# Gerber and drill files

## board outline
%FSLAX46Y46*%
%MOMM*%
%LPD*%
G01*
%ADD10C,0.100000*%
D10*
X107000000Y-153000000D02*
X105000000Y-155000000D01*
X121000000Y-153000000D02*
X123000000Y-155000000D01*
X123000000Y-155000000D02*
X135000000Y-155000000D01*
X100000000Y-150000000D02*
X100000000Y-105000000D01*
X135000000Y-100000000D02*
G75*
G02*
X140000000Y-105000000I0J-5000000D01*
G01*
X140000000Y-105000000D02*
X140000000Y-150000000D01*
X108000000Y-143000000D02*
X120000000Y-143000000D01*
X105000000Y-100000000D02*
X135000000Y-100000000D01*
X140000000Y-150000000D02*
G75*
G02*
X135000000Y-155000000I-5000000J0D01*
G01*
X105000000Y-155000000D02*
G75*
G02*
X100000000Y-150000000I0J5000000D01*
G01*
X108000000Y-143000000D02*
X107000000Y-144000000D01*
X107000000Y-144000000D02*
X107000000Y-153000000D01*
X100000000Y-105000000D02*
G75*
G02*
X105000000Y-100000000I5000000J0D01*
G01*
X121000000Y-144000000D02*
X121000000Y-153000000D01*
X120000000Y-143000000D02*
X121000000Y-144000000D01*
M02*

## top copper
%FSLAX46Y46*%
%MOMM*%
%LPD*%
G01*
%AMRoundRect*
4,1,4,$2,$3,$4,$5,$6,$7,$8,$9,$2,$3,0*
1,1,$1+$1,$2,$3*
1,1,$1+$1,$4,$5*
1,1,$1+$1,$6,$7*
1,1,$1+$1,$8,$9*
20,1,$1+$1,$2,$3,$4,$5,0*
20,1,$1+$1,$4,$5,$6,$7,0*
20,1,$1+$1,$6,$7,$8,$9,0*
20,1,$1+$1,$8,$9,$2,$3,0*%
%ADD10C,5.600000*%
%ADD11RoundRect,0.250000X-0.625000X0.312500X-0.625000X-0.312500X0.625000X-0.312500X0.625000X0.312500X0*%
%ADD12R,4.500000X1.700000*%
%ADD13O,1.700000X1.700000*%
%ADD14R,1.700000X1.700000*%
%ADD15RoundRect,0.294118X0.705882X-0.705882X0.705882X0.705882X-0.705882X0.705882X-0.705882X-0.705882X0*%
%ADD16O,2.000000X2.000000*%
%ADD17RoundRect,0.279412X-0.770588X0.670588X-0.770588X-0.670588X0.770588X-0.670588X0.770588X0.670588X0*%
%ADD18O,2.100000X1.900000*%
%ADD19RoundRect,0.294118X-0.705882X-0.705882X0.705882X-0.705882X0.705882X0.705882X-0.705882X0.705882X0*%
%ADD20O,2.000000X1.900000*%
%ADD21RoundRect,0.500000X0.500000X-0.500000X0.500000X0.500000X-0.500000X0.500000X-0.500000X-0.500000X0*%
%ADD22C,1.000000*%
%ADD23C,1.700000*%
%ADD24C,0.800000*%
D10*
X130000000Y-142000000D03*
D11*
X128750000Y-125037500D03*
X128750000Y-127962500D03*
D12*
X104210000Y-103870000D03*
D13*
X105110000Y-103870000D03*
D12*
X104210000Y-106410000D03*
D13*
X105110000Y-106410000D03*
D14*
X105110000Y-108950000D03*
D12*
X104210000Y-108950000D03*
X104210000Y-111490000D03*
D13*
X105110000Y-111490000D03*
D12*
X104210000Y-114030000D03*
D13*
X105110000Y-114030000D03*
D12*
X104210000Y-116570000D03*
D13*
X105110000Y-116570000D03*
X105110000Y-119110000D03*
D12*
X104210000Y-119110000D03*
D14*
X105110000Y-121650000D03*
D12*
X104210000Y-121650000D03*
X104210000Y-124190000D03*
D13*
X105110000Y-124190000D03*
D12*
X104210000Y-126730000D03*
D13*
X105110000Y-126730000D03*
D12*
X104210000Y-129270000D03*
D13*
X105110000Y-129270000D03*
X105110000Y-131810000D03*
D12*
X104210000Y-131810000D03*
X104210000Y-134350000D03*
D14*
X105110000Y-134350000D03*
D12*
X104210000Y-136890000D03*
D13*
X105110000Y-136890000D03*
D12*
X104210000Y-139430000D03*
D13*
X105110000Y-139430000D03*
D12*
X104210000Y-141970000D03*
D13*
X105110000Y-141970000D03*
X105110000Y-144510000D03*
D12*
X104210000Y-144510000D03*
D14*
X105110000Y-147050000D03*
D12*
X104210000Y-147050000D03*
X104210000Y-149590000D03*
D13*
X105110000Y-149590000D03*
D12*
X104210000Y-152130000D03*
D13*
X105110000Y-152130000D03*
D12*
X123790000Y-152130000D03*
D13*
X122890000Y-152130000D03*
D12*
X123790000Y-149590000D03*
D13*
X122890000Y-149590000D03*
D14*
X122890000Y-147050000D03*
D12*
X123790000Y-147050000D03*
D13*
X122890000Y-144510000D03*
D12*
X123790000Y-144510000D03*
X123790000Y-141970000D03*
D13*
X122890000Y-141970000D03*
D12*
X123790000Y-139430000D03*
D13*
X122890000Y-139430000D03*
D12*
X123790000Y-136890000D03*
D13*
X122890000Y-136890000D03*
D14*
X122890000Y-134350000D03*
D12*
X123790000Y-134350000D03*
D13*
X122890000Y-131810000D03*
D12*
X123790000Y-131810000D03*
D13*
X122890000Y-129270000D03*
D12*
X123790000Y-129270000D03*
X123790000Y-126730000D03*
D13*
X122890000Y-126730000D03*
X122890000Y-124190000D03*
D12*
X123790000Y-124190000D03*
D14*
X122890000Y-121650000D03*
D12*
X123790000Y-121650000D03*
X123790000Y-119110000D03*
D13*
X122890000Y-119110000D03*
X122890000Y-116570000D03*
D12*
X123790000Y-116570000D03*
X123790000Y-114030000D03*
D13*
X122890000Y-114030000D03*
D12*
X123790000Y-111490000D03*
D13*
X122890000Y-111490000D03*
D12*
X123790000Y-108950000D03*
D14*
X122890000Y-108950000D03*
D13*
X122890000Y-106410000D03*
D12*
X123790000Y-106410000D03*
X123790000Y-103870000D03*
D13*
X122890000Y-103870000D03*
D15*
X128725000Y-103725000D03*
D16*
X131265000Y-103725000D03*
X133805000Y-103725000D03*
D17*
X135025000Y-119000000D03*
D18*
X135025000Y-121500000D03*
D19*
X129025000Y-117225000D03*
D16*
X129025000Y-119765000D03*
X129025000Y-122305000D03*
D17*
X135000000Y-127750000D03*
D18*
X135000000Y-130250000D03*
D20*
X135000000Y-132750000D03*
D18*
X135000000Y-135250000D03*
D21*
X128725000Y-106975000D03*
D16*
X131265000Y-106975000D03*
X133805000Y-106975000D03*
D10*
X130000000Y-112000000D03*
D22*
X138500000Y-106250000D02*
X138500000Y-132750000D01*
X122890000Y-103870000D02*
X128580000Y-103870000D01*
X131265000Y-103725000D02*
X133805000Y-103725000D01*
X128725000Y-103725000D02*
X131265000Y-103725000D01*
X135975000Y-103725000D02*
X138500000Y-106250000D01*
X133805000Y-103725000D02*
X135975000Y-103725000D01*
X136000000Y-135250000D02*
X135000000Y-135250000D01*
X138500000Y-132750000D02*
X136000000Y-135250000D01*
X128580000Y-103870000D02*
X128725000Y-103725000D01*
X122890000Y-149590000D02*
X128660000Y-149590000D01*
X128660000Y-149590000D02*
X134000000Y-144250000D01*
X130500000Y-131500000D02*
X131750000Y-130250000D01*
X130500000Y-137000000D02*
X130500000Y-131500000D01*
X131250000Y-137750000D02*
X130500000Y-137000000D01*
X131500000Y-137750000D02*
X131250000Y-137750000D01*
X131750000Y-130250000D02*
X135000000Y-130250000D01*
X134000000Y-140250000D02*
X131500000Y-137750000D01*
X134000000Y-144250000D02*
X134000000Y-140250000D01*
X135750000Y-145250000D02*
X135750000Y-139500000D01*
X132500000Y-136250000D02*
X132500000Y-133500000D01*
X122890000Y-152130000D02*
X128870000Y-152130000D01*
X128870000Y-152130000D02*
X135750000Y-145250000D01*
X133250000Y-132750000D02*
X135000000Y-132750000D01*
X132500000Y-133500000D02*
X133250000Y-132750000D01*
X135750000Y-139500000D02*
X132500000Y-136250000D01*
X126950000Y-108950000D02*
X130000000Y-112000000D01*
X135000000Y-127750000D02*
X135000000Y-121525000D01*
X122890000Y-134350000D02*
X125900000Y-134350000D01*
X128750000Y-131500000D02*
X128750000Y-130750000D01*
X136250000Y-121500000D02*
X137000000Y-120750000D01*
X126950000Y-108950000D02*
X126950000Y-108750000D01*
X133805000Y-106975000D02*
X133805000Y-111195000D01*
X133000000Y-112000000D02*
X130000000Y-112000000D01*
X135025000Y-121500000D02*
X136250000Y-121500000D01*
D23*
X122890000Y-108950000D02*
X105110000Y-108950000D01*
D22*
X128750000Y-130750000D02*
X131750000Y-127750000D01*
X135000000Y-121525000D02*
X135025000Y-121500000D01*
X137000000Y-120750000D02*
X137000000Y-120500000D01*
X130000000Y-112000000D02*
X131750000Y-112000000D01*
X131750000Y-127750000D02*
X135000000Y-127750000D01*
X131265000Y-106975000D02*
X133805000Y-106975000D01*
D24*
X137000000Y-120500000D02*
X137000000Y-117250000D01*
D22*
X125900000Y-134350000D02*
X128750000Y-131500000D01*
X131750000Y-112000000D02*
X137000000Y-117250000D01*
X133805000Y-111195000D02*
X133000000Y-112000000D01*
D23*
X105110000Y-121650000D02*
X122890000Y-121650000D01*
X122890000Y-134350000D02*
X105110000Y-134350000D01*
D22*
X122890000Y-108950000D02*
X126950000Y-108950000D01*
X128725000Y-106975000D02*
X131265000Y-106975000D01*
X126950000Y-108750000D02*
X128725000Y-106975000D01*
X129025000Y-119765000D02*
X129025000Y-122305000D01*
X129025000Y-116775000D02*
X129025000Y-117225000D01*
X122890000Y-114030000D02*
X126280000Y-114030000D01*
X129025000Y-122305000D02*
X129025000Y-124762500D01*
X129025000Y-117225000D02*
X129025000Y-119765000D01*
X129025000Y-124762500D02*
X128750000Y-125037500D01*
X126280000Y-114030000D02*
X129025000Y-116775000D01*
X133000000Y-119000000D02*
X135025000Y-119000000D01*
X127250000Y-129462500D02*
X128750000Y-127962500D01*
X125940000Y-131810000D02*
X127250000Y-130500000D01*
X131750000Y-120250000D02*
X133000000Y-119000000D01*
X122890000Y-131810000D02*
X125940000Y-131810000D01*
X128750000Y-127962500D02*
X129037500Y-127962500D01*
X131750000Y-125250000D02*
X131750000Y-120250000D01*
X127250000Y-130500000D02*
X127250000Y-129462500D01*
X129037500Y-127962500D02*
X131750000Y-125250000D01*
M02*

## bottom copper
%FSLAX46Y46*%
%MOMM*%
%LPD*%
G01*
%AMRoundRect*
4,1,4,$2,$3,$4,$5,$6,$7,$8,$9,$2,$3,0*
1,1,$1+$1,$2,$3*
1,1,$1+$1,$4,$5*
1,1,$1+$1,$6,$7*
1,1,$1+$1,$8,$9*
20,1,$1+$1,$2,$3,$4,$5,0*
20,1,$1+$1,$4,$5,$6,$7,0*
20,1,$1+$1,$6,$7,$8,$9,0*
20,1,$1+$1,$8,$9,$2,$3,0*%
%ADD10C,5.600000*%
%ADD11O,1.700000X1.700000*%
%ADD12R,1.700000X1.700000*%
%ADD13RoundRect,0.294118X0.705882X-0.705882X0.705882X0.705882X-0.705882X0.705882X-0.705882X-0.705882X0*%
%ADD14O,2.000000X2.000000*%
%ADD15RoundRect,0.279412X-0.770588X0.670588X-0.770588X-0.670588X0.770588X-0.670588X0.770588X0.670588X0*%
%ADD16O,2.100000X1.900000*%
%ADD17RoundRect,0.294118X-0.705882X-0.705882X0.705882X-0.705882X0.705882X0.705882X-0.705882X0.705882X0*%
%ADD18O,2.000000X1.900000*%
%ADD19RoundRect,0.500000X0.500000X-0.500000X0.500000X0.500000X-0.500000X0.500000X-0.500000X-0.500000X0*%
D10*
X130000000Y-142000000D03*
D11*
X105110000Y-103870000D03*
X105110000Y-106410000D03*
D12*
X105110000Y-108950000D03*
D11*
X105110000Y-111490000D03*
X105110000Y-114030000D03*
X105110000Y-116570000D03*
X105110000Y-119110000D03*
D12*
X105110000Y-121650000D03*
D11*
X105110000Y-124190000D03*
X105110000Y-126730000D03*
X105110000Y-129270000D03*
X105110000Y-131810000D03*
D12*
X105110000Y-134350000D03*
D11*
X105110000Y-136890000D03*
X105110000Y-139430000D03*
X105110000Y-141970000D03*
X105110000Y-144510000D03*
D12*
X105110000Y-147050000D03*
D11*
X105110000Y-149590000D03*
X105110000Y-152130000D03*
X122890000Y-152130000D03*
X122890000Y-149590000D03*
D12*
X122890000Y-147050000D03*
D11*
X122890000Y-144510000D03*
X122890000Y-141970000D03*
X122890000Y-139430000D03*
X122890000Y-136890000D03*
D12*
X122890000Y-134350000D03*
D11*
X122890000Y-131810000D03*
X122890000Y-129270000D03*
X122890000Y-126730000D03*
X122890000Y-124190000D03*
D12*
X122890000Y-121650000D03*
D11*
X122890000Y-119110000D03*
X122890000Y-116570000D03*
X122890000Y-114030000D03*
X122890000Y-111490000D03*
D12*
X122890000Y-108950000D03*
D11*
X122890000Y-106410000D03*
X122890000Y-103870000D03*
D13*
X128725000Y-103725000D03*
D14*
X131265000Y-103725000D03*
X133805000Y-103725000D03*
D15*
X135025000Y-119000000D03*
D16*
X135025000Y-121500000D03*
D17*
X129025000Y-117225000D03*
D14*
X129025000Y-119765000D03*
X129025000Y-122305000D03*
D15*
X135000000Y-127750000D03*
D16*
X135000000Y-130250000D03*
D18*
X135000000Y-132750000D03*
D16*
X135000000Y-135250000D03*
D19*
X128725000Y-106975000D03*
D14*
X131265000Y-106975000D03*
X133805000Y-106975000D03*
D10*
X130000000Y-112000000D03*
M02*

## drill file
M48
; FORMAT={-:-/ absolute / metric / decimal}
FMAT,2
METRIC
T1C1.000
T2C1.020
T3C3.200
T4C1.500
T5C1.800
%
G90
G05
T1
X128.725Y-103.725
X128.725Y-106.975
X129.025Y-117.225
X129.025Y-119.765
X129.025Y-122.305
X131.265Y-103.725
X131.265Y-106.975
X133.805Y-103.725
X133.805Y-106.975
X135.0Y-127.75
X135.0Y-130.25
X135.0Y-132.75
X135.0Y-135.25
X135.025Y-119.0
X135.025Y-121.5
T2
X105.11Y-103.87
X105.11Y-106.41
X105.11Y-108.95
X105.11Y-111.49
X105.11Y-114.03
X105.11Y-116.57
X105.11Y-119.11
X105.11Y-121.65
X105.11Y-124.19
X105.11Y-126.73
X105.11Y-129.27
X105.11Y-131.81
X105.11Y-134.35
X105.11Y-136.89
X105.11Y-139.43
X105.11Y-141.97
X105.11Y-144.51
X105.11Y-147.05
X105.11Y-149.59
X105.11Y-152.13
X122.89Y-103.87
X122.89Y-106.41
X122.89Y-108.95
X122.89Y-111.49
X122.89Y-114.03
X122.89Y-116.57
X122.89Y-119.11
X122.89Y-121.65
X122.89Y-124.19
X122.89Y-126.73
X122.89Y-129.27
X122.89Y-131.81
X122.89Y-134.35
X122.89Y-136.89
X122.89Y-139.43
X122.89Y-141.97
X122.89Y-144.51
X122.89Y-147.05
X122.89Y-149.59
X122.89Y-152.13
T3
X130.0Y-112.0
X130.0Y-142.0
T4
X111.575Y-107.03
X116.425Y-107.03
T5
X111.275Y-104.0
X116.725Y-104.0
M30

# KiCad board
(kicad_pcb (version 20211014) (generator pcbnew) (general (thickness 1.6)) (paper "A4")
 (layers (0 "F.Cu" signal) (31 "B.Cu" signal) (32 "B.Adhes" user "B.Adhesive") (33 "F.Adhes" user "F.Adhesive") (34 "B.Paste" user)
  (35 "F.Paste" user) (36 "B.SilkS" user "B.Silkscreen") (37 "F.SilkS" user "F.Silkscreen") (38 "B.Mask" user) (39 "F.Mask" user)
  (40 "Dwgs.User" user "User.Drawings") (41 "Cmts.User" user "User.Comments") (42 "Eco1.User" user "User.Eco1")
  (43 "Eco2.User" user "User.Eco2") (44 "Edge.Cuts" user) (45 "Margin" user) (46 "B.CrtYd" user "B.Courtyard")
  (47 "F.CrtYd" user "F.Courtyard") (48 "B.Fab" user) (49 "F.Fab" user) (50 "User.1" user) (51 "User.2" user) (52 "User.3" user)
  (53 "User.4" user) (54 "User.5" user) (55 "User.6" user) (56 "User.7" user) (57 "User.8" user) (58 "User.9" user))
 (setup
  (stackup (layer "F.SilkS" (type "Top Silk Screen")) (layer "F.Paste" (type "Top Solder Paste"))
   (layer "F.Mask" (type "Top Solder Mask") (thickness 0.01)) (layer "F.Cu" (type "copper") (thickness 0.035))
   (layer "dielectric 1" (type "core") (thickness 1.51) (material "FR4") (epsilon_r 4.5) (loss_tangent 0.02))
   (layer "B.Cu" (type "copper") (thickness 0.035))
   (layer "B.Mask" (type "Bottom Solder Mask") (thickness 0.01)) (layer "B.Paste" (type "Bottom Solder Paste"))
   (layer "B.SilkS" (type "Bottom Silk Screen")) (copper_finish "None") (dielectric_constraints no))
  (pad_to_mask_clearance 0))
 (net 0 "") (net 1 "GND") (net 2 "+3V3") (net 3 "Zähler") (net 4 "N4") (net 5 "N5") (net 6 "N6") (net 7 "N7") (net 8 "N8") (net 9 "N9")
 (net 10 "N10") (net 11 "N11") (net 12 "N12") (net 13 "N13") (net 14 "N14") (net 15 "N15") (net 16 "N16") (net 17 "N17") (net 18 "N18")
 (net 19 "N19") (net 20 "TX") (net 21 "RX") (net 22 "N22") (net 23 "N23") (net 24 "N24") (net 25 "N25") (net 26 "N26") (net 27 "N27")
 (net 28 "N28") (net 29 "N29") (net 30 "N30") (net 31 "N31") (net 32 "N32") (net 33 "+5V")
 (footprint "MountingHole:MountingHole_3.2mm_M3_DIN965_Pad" (layer "F.Cu") (at 130 142)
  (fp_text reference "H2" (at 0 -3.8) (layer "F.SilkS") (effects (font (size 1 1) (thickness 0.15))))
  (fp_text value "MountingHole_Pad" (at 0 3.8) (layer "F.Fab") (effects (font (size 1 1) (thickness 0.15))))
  (pad "1" thru_hole circle (at 0 0) (size 5.6 5.6) (drill 3.2) (layers *.Cu *.Mask) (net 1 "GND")))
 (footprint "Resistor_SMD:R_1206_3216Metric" (layer "F.Cu") (at 128.75 126.5 -90)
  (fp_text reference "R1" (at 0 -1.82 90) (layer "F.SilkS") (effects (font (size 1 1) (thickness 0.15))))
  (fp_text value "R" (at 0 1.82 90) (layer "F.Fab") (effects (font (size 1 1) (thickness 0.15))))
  (pad "1" smd roundrect (at -1.4625 0 270) (size 1.125 1.75) (layers "F.Cu" "F.Paste" "F.Mask") (roundrect_rratio 0.222222) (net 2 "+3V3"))
  (pad "2" smd roundrect (at 1.4625 0 270) (size 1.125 1.75) (layers "F.Cu" "F.Paste" "F.Mask") (roundrect_rratio 0.222222) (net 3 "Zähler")))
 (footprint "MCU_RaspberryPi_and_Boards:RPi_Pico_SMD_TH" (layer "F.Cu") (at 114 128)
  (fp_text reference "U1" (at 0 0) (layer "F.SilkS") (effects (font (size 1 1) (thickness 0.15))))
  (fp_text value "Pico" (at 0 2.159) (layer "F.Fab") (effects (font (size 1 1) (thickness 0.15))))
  (pad "" np_thru_hole oval (at -2.425 -20.97) (size 1.5 1.5) (drill 1.5) (layers *.Cu *.Mask))
  (pad "" np_thru_hole oval (at 2.425 -20.97) (size 1.5 1.5) (drill 1.5) (layers *.Cu *.Mask))
  (pad "" np_thru_hole oval (at -2.725 -24) (size 1.8 1.8) (drill 1.8) (layers *.Cu *.Mask))
  (pad "" np_thru_hole oval (at 2.725 -24) (size 1.8 1.8) (drill 1.8) (layers *.Cu *.Mask))
  (pad "1" smd rect (at -8.89 -24.13) (size 4.5 1.7) (drill (offset -0.9 0)) (layers "F.Cu" "F.Mask") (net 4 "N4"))
  (pad "1" thru_hole oval (at -8.89 -24.13) (size 1.7 1.7) (drill 1.02) (layers *.Cu *.Mask) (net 4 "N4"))
  (pad "2" smd rect (at -8.89 -21.59) (size 4.5 1.7) (drill (offset -0.9 0)) (layers "F.Cu" "F.Mask") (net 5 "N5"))
  (pad "2" thru_hole oval (at -8.89 -21.59) (size 1.7 1.7) (drill 1.02) (layers *.Cu *.Mask) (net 5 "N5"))
  (pad "3" thru_hole rect (at -8.89 -19.05) (size 1.7 1.7) (drill 1.02) (layers *.Cu *.Mask) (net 1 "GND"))
  (pad "3" smd rect (at -8.89 -19.05) (size 4.5 1.7) (drill (offset -0.9 0)) (layers "F.Cu" "F.Mask") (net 1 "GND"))
  (pad "4" smd rect (at -8.89 -16.51) (size 4.5 1.7) (drill (offset -0.9 0)) (layers "F.Cu" "F.Mask") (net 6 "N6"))
  (pad "4" thru_hole oval (at -8.89 -16.51) (size 1.7 1.7) (drill 1.02) (layers *.Cu *.Mask) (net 6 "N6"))
  (pad "5" smd rect (at -8.89 -13.97) (size 4.5 1.7) (drill (offset -0.9 0)) (layers "F.Cu" "F.Mask") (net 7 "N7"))
  (pad "5" thru_hole oval (at -8.89 -13.97) (size 1.7 1.7) (drill 1.02) (layers *.Cu *.Mask) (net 7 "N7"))
  (pad "6" smd rect (at -8.89 -11.43) (size 4.5 1.7) (drill (offset -0.9 0)) (layers "F.Cu" "F.Mask") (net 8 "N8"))
  (pad "6" thru_hole oval (at -8.89 -11.43) (size 1.7 1.7) (drill 1.02) (layers *.Cu *.Mask) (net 8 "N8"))
  (pad "7" thru_hole oval (at -8.89 -8.89) (size 1.7 1.7) (drill 1.02) (layers *.Cu *.Mask) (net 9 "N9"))
  (pad "7" smd rect (at -8.89 -8.89) (size 4.5 1.7) (drill (offset -0.9 0)) (layers "F.Cu" "F.Mask") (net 9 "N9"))
  (pad "8" thru_hole rect (at -8.89 -6.35) (size 1.7 1.7) (drill 1.02) (layers *.Cu *.Mask) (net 1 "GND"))
  (pad "8" smd rect (at -8.89 -6.35) (size 4.5 1.7) (drill (offset -0.9 0)) (layers "F.Cu" "F.Mask") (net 1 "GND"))
  (pad "9" smd rect (at -8.89 -3.81) (size 4.5 1.7) (drill (offset -0.9 0)) (layers "F.Cu" "F.Mask") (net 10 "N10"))
  (pad "9" thru_hole oval (at -8.89 -3.81) (size 1.7 1.7) (drill 1.02) (layers *.Cu *.Mask) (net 10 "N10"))
  (pad "10" smd rect (at -8.89 -1.27) (size 4.5 1.7) (drill (offset -0.9 0)) (layers "F.Cu" "F.Mask") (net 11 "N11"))
  (pad "10" thru_hole oval (at -8.89 -1.27) (size 1.7 1.7) (drill 1.02) (layers *.Cu *.Mask) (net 11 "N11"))
  (pad "11" smd rect (at -8.89 1.27) (size 4.5 1.7) (drill (offset -0.9 0)) (layers "F.Cu" "F.Mask") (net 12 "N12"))
  (pad "11" thru_hole oval (at -8.89 1.27) (size 1.7 1.7) (drill 1.02) (layers *.Cu *.Mask) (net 12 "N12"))
  (pad "12" thru_hole oval (at -8.89 3.81) (size 1.7 1.7) (drill 1.02) (layers *.Cu *.Mask) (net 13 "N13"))
  (pad "12" smd rect (at -8.89 3.81) (size 4.5 1.7) (drill (offset -0.9 0)) (layers "F.Cu" "F.Mask") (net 13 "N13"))
  (pad "13" smd rect (at -8.89 6.35) (size 4.5 1.7) (drill (offset -0.9 0)) (layers "F.Cu" "F.Mask") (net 1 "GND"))
  (pad "13" thru_hole rect (at -8.89 6.35) (size 1.7 1.7) (drill 1.02) (layers *.Cu *.Mask) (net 1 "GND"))
  (pad "14" smd rect (at -8.89 8.89) (size 4.5 1.7) (drill (offset -0.9 0)) (layers "F.Cu" "F.Mask") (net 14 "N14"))
  (pad "14" thru_hole oval (at -8.89 8.89) (size 1.7 1.7) (drill 1.02) (layers *.Cu *.Mask) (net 14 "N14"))
  (pad "15" smd rect (at -8.89 11.43) (size 4.5 1.7) (drill (offset -0.9 0)) (layers "F.Cu" "F.Mask") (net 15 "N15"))
  (pad "15" thru_hole oval (at -8.89 11.43) (size 1.7 1.7) (drill 1.02) (layers *.Cu *.Mask) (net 15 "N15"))
  (pad "16" smd rect (at -8.89 13.97) (size 4.5 1.7) (drill (offset -0.9 0)) (layers "F.Cu" "F.Mask") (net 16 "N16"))
  (pad "16" thru_hole oval (at -8.89 13.97) (size 1.7 1.7) (drill 1.02) (layers *.Cu *.Mask) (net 16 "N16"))
  (pad "17" thru_hole oval (at -8.89 16.51) (size 1.7 1.7) (drill 1.02) (layers *.Cu *.Mask) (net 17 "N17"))
  (pad "17" smd rect (at -8.89 16.51) (size 4.5 1.7) (drill (offset -0.9 0)) (layers "F.Cu" "F.Mask") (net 17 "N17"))
  (pad "18" thru_hole rect (at -8.89 19.05) (size 1.7 1.7) (drill 1.02) (layers *.Cu *.Mask) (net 1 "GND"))
  (pad "18" smd rect (at -8.89 19.05) (size 4.5 1.7) (drill (offset -0.9 0)) (layers "F.Cu" "F.Mask") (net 1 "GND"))
  (pad "19" smd rect (at -8.89 21.59) (size 4.5 1.7) (drill (offset -0.9 0)) (layers "F.Cu" "F.Mask") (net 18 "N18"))
  (pad "19" thru_hole oval (at -8.89 21.59) (size 1.7 1.7) (drill 1.02) (layers *.Cu *.Mask) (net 18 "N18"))
  (pad "20" smd rect (at -8.89 24.13) (size 4.5 1.7) (drill (offset -0.9 0)) (layers "F.Cu" "F.Mask") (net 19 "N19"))
  (pad "20" thru_hole oval (at -8.89 24.13) (size 1.7 1.7) (drill 1.02) (layers *.Cu *.Mask) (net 19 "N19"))
  (pad "21" smd rect (at 8.89 24.13) (size 4.5 1.7) (drill (offset 0.9 0)) (layers "F.Cu" "F.Mask") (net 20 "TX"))
  (pad "21" thru_hole oval (at 8.89 24.13) (size 1.7 1.7) (drill 1.02) (layers *.Cu *.Mask) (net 20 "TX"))
  (pad "22" smd rect (at 8.89 21.59) (size 4.5 1.7) (drill (offset 0.9 0)) (layers "F.Cu" "F.Mask") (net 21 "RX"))
  (pad "22" thru_hole oval (at 8.89 21.59) (size 1.7 1.7) (drill 1.02) (layers *.Cu *.Mask) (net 21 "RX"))
  (pad "23" thru_hole rect (at 8.89 19.05) (size 1.7 1.7) (drill 1.02) (layers *.Cu *.Mask) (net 1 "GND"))
  (pad "23" smd rect (at 8.89 19.05) (size 4.5 1.7) (drill (offset 0.9 0)) (layers "F.Cu" "F.Mask") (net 1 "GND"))
  (pad "24" thru_hole oval (at 8.89 16.51) (size 1.7 1.7) (drill 1.02) (layers *.Cu *.Mask) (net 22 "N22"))
  (pad "24" smd rect (at 8.89 16.51) (size 4.5 1.7) (drill (offset 0.9 0)) (layers "F.Cu" "F.Mask") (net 22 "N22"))
  (pad "25" smd rect (at 8.89 13.97) (size 4.5 1.7) (drill (offset 0.9 0)) (layers "F.Cu" "F.Mask") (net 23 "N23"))
  (pad "25" thru_hole oval (at 8.89 13.97) (size 1.7 1.7) (drill 1.02) (layers *.Cu *.Mask) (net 23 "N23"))
  (pad "26" smd rect (at 8.89 11.43) (size 4.5 1.7) (drill (offset 0.9 0)) (layers "F.Cu" "F.Mask") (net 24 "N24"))
  (pad "26" thru_hole oval (at 8.89 11.43) (size 1.7 1.7) (drill 1.02) (layers *.Cu *.Mask) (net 24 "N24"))
  (pad "27" smd rect (at 8.89 8.89) (size 4.5 1.7) (drill (offset 0.9 0)) (layers "F.Cu" "F.Mask") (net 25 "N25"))
  (pad "27" thru_hole oval (at 8.89 8.89) (size 1.7 1.7) (drill 1.02) (layers *.Cu *.Mask) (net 25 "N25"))
  (pad "28" thru_hole rect (at 8.89 6.35) (size 1.7 1.7) (drill 1.02) (layers *.Cu *.Mask) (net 1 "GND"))
  (pad "28" smd rect (at 8.89 6.35) (size 4.5 1.7) (drill (offset 0.9 0)) (layers "F.Cu" "F.Mask") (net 1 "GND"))
  (pad "29" thru_hole oval (at 8.89 3.81) (size 1.7 1.7) (drill 1.02) (layers *.Cu *.Mask) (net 3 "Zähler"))
  (pad "29" smd rect (at 8.89 3.81) (size 4.5 1.7) (drill (offset 0.9 0)) (layers "F.Cu" "F.Mask") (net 3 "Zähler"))
  (pad "30" thru_hole oval (at 8.89 1.27) (size 1.7 1.7) (drill 1.02) (layers *.Cu *.Mask) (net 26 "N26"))
  (pad "30" smd rect (at 8.89 1.27) (size 4.5 1.7) (drill (offset 0.9 0)) (layers "F.Cu" "F.Mask") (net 26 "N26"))
  (pad "31" smd rect (at 8.89 -1.27) (size 4.5 1.7) (drill (offset 0.9 0)) (layers "F.Cu" "F.Mask") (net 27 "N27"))
  (pad "31" thru_hole oval (at 8.89 -1.27) (size 1.7 1.7) (drill 1.02) (layers *.Cu *.Mask) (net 27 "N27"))
  (pad "32" thru_hole oval (at 8.89 -3.81) (size 1.7 1.7) (drill 1.02) (layers *.Cu *.Mask) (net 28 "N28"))
  (pad "32" smd rect (at 8.89 -3.81) (size 4.5 1.7) (drill (offset 0.9 0)) (layers "F.Cu" "F.Mask") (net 28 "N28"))
  (pad "33" thru_hole rect (at 8.89 -6.35) (size 1.7 1.7) (drill 1.02) (layers *.Cu *.Mask) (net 1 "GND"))
  (pad "33" smd rect (at 8.89 -6.35) (size 4.5 1.7) (drill (offset 0.9 0)) (layers "F.Cu" "F.Mask") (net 1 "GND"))
  (pad "34" smd rect (at 8.89 -8.89) (size 4.5 1.7) (drill (offset 0.9 0)) (layers "F.Cu" "F.Mask") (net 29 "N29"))
  (pad "34" thru_hole oval (at 8.89 -8.89) (size 1.7 1.7) (drill 1.02) (layers *.Cu *.Mask) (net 29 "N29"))
  (pad "35" thru_hole oval (at 8.89 -11.43) (size 1.7 1.7) (drill 1.02) (layers *.Cu *.Mask) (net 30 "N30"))
  (pad "35" smd rect (at 8.89 -11.43) (size 4.5 1.7) (drill (offset 0.9 0)) (layers "F.Cu" "F.Mask") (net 30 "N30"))
  (pad "36" smd rect (at 8.89 -13.97) (size 4.5 1.7) (drill (offset 0.9 0)) (layers "F.Cu" "F.Mask") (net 2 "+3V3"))
  (pad "36" thru_hole oval (at 8.89 -13.97) (size 1.7 1.7) (drill 1.02) (layers *.Cu *.Mask) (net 2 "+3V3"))
  (pad "37" smd rect (at 8.89 -16.51) (size 4.5 1.7) (drill (offset 0.9 0)) (layers "F.Cu" "F.Mask") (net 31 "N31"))
  (pad "37" thru_hole oval (at 8.89 -16.51) (size 1.7 1.7) (drill 1.02) (layers *.Cu *.Mask) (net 31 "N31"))
  (pad "38" smd rect (at 8.89 -19.05) (size 4.5 1.7) (drill (offset 0.9 0)) (layers "F.Cu" "F.Mask") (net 1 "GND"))
  (pad "38" thru_hole rect (at 8.89 -19.05) (size 1.7 1.7) (drill 1.02) (layers *.Cu *.Mask) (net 1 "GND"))
  (pad "39" thru_hole oval (at 8.89 -21.59) (size 1.7 1.7) (drill 1.02) (layers *.Cu *.Mask) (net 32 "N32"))
  (pad "39" smd rect (at 8.89 -21.59) (size 4.5 1.7) (drill (offset 0.9 0)) (layers "F.Cu" "F.Mask") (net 32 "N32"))
  (pad "40" smd rect (at 8.89 -24.13) (size 4.5 1.7) (drill (offset 0.9 0)) (layers "F.Cu" "F.Mask") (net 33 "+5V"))
  (pad "40" thru_hole oval (at 8.89 -24.13) (size 1.7 1.7) (drill 1.02) (layers *.Cu *.Mask) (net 33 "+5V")))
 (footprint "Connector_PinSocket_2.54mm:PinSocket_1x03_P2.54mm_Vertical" (layer "F.Cu") (at 128.725 103.725 90)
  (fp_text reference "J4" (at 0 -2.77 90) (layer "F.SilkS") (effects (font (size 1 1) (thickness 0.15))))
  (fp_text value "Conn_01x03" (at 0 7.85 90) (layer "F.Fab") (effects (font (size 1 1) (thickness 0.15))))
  (pad "1" thru_hole roundrect (at 0 0 90) (size 2 2) (drill 1) (layers *.Cu *.Mask) (roundrect_rratio 0.147059) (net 33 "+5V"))
  (pad "2" thru_hole oval (at 0 2.54 90) (size 2 2) (drill 1) (layers *.Cu *.Mask) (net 33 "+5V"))
  (pad "3" thru_hole oval (at 0 5.08 90) (size 2 2) (drill 1) (layers *.Cu *.Mask) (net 33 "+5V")))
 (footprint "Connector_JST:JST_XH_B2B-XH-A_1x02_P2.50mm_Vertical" (layer "F.Cu") (at 135.025 119 -90)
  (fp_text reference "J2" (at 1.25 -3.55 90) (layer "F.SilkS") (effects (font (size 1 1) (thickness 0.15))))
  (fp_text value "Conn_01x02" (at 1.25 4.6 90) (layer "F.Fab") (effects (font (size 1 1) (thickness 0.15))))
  (pad "1" thru_hole roundrect (at 0 0 270) (size 1.9 2.1) (drill 1) (layers *.Cu *.Mask) (roundrect_rratio 0.147059) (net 3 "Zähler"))
  (pad "2" thru_hole oval (at 2.5 0 270) (size 1.9 2.1) (drill 1) (layers *.Cu *.Mask) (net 1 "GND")))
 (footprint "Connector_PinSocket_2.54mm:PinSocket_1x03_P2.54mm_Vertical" (layer "F.Cu") (at 129.025 117.225)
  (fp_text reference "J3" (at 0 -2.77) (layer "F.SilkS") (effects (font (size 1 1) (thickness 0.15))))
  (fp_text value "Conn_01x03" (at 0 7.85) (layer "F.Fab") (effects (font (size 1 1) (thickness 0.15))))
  (pad "1" thru_hole roundrect (at 0 0) (size 2 2) (drill 1) (layers *.Cu *.Mask) (roundrect_rratio 0.147059) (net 2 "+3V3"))
  (pad "2" thru_hole oval (at 0 2.54) (size 2 2) (drill 1) (layers *.Cu *.Mask) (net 2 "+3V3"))
  (pad "3" thru_hole oval (at 0 5.08) (size 2 2) (drill 1) (layers *.Cu *.Mask) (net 2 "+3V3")))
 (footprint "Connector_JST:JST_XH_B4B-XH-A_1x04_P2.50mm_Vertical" (layer "F.Cu") (at 135 127.75 -90)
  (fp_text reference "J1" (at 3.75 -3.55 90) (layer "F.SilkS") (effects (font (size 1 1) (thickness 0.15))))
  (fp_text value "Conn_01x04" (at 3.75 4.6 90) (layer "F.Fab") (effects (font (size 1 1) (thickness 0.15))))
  (pad "1" thru_hole roundrect (at 0 0 270) (size 1.9 2.1) (drill 1) (layers *.Cu *.Mask) (roundrect_rratio 0.147059) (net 1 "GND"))
  (pad "2" thru_hole oval (at 2.5 0 270) (size 1.9 2.1) (drill 1) (layers *.Cu *.Mask) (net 21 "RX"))
  (pad "3" thru_hole oval (at 5 0 270) (size 1.9 2) (drill 1) (layers *.Cu *.Mask) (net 20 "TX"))
  (pad "4" thru_hole oval (at 7.5 0 270) (size 1.9 2.1) (drill 1) (layers *.Cu *.Mask) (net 33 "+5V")))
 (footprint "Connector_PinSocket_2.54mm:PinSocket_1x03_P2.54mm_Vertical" (layer "F.Cu") (at 128.725 106.975 90)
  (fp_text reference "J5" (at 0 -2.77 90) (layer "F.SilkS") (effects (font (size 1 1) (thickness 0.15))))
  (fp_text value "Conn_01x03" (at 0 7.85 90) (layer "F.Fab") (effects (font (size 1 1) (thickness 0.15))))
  (pad "1" thru_hole roundrect (at 0 0 90) (size 2 2) (drill 1) (layers *.Cu *.Mask) (roundrect_rratio 0.25) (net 1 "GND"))
  (pad "2" thru_hole oval (at 0 2.54 90) (size 2 2) (drill 1) (layers *.Cu *.Mask) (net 1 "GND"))
  (pad "3" thru_hole oval (at 0 5.08 90) (size 2 2) (drill 1) (layers *.Cu *.Mask) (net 1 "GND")))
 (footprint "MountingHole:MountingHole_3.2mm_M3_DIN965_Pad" (layer "F.Cu") (at 130 112)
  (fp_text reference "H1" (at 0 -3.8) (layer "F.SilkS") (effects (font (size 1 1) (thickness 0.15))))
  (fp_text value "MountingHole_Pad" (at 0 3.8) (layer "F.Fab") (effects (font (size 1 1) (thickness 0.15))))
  (pad "1" thru_hole circle (at 0 0) (size 5.6 5.6) (drill 3.2) (layers *.Cu *.Mask) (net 1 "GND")))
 (gr_line (start 107 153) (end 105 155) (layer "Edge.Cuts") (width 0.1))
 (gr_line (start 121 153) (end 123 155) (layer "Edge.Cuts") (width 0.1))
 (gr_line (start 123 155) (end 135 155) (layer "Edge.Cuts") (width 0.1))
 (gr_line (start 100 150) (end 100 105) (layer "Edge.Cuts") (width 0.1))
 (gr_arc (start 135 100) (mid 138.535534 101.464466) (end 140 105) (layer "Edge.Cuts") (width 0.1))
 (gr_line (start 140 105) (end 140 150) (layer "Edge.Cuts") (width 0.1))
 (gr_line (start 108 143) (end 120 143) (layer "Edge.Cuts") (width 0.1))
 (gr_line (start 105 100) (end 135 100) (layer "Edge.Cuts") (width 0.1))
 (gr_arc (start 140 150) (mid 138.535534 153.535534) (end 135 155) (layer "Edge.Cuts") (width 0.1))
 (gr_arc (start 105 155) (mid 101.464466 153.535534) (end 100 150) (layer "Edge.Cuts") (width 0.1))
 (gr_line (start 108 143) (end 107 144) (layer "Edge.Cuts") (width 0.1))
 (gr_line (start 107 144) (end 107 153) (layer "Edge.Cuts") (width 0.1))
 (gr_arc (start 100 105) (mid 101.464466 101.464466) (end 105 100) (layer "Edge.Cuts") (width 0.1))
 (gr_line (start 121 144) (end 121 153) (layer "Edge.Cuts") (width 0.1))
 (gr_line (start 120 143) (end 121 144) (layer "Edge.Cuts") (width 0.1))
 (segment (start 138.5 106.25) (end 138.5 132.75) (width 1) (layer "F.Cu") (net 33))
 (segment (start 122.89 103.87) (end 128.58 103.87) (width 1) (layer "F.Cu") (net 33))
 (segment (start 131.265 103.725) (end 133.805 103.725) (width 1) (layer "F.Cu") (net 33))
 (segment (start 128.725 103.725) (end 131.265 103.725) (width 1) (layer "F.Cu") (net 33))
 (segment (start 135.975 103.725) (end 138.5 106.25) (width 1) (layer "F.Cu") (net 33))
 (segment (start 133.805 103.725) (end 135.975 103.725) (width 1) (layer "F.Cu") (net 33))
 (segment (start 136 135.25) (end 135 135.25) (width 1) (layer "F.Cu") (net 33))
 (segment (start 138.5 132.75) (end 136 135.25) (width 1) (layer "F.Cu") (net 33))
 (segment (start 128.58 103.87) (end 128.725 103.725) (width 1) (layer "F.Cu") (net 33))
 (segment (start 122.89 149.59) (end 128.66 149.59) (width 1) (layer "F.Cu") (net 21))
 (segment (start 128.66 149.59) (end 134 144.25) (width 1) (layer "F.Cu") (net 21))
 (segment (start 130.5 131.5) (end 131.75 130.25) (width 1) (layer "F.Cu") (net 21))
 (segment (start 130.5 137) (end 130.5 131.5) (width 1) (layer "F.Cu") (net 21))
 (segment (start 131.25 137.75) (end 130.5 137) (width 1) (layer "F.Cu") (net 21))
 (segment (start 131.5 137.75) (end 131.25 137.75) (width 1) (layer "F.Cu") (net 21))
 (segment (start 131.75 130.25) (end 135 130.25) (width 1) (layer "F.Cu") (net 21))
 (segment (start 134 140.25) (end 131.5 137.75) (width 1) (layer "F.Cu") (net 21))
 (segment (start 134 144.25) (end 134 140.25) (width 1) (layer "F.Cu") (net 21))
 (segment (start 135.75 145.25) (end 135.75 139.5) (width 1) (layer "F.Cu") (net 20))
 (segment (start 132.5 136.25) (end 132.5 133.5) (width 1) (layer "F.Cu") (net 20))
 (segment (start 122.89 152.13) (end 128.87 152.13) (width 1) (layer "F.Cu") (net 20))
 (segment (start 128.87 152.13) (end 135.75 145.25) (width 1) (layer "F.Cu") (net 20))
 (segment (start 133.25 132.75) (end 135 132.75) (width 1) (layer "F.Cu") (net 20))
 (segment (start 132.5 133.5) (end 133.25 132.75) (width 1) (layer "F.Cu") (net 20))
 (segment (start 135.75 139.5) (end 132.5 136.25) (width 1) (layer "F.Cu") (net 20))
 (segment (start 126.95 108.95) (end 130 112) (width 1) (layer "F.Cu") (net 1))
 (segment (start 135 127.75) (end 135 121.525) (width 1) (layer "F.Cu") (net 1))
 (segment (start 122.89 134.35) (end 125.9 134.35) (width 1) (layer "F.Cu") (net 1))
 (segment (start 128.75 131.5) (end 128.75 130.75) (width 1) (layer "F.Cu") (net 1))
 (segment (start 136.25 121.5) (end 137 120.75) (width 1) (layer "F.Cu") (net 1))
 (segment (start 126.95 108.95) (end 126.95 108.75) (width 1) (layer "F.Cu") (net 1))
 (segment (start 133.805 106.975) (end 133.805 111.195) (width 1) (layer "F.Cu") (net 1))
 (segment (start 133 112) (end 130 112) (width 1) (layer "F.Cu") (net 1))
 (segment (start 135.025 121.5) (end 136.25 121.5) (width 1) (layer "F.Cu") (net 1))
 (segment (start 122.89 108.95) (end 105.11 108.95) (width 1.7) (layer "F.Cu") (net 1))
 (segment (start 128.75 130.75) (end 131.75 127.75) (width 1) (layer "F.Cu") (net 1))
 (segment (start 135 121.525) (end 135.025 121.5) (width 1) (layer "F.Cu") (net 1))
 (segment (start 137 120.75) (end 137 120.5) (width 1) (layer "F.Cu") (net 1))
 (segment (start 130 112) (end 131.75 112) (width 1) (layer "F.Cu") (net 1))
 (segment (start 131.75 127.75) (end 135 127.75) (width 1) (layer "F.Cu") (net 1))
 (segment (start 131.265 106.975) (end 133.805 106.975) (width 1) (layer "F.Cu") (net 1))
 (segment (start 137 120.5) (end 137 117.25) (width 0.8) (layer "F.Cu") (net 1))
 (segment (start 125.9 134.35) (end 128.75 131.5) (width 1) (layer "F.Cu") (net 1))
 (segment (start 131.75 112) (end 137 117.25) (width 1) (layer "F.Cu") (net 1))
 (segment (start 133.805 111.195) (end 133 112) (width 1) (layer "F.Cu") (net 1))
 (segment (start 105.11 121.65) (end 122.89 121.65) (width 1.7) (layer "F.Cu") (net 1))
 (segment (start 122.89 134.35) (end 105.11 134.35) (width 1.7) (layer "F.Cu") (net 1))
 (segment (start 122.89 108.95) (end 126.95 108.95) (width 1) (layer "F.Cu") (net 1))
 (segment (start 128.725 106.975) (end 131.265 106.975) (width 1) (layer "F.Cu") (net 1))
 (segment (start 126.95 108.75) (end 128.725 106.975) (width 1) (layer "F.Cu") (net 1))
 (segment (start 129.025 119.765) (end 129.025 122.305) (width 1) (layer "F.Cu") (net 2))
 (segment (start 129.025 116.775) (end 129.025 117.225) (width 1) (layer "F.Cu") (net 2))
 (segment (start 122.89 114.03) (end 126.28 114.03) (width 1) (layer "F.Cu") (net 2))
 (segment (start 129.025 122.305) (end 129.025 124.7625) (width 1) (layer "F.Cu") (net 2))
 (segment (start 129.025 117.225) (end 129.025 119.765) (width 1) (layer "F.Cu") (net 2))
 (segment (start 129.025 124.7625) (end 128.75 125.0375) (width 1) (layer "F.Cu") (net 2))
 (segment (start 126.28 114.03) (end 129.025 116.775) (width 1) (layer "F.Cu") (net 2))
 (segment (start 133 119) (end 135.025 119) (width 1) (layer "F.Cu") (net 3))
 (segment (start 127.25 129.4625) (end 128.75 127.9625) (width 1) (layer "F.Cu") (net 3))
 (segment (start 125.94 131.81) (end 127.25 130.5) (width 1) (layer "F.Cu") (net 3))
 (segment (start 131.75 120.25) (end 133 119) (width 1) (layer "F.Cu") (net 3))
 (segment (start 122.89 131.81) (end 125.94 131.81) (width 1) (layer "F.Cu") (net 3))
 (segment (start 128.75 127.9625) (end 129.0375 127.9625) (width 1) (layer "F.Cu") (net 3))
 (segment (start 131.75 125.25) (end 131.75 120.25) (width 1) (layer "F.Cu") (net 3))
 (segment (start 127.25 130.5) (end 127.25 129.4625) (width 1) (layer "F.Cu") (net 3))
 (segment (start 129.0375 127.9625) (end 131.75 125.25) (width 1) (layer "F.Cu") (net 3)))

